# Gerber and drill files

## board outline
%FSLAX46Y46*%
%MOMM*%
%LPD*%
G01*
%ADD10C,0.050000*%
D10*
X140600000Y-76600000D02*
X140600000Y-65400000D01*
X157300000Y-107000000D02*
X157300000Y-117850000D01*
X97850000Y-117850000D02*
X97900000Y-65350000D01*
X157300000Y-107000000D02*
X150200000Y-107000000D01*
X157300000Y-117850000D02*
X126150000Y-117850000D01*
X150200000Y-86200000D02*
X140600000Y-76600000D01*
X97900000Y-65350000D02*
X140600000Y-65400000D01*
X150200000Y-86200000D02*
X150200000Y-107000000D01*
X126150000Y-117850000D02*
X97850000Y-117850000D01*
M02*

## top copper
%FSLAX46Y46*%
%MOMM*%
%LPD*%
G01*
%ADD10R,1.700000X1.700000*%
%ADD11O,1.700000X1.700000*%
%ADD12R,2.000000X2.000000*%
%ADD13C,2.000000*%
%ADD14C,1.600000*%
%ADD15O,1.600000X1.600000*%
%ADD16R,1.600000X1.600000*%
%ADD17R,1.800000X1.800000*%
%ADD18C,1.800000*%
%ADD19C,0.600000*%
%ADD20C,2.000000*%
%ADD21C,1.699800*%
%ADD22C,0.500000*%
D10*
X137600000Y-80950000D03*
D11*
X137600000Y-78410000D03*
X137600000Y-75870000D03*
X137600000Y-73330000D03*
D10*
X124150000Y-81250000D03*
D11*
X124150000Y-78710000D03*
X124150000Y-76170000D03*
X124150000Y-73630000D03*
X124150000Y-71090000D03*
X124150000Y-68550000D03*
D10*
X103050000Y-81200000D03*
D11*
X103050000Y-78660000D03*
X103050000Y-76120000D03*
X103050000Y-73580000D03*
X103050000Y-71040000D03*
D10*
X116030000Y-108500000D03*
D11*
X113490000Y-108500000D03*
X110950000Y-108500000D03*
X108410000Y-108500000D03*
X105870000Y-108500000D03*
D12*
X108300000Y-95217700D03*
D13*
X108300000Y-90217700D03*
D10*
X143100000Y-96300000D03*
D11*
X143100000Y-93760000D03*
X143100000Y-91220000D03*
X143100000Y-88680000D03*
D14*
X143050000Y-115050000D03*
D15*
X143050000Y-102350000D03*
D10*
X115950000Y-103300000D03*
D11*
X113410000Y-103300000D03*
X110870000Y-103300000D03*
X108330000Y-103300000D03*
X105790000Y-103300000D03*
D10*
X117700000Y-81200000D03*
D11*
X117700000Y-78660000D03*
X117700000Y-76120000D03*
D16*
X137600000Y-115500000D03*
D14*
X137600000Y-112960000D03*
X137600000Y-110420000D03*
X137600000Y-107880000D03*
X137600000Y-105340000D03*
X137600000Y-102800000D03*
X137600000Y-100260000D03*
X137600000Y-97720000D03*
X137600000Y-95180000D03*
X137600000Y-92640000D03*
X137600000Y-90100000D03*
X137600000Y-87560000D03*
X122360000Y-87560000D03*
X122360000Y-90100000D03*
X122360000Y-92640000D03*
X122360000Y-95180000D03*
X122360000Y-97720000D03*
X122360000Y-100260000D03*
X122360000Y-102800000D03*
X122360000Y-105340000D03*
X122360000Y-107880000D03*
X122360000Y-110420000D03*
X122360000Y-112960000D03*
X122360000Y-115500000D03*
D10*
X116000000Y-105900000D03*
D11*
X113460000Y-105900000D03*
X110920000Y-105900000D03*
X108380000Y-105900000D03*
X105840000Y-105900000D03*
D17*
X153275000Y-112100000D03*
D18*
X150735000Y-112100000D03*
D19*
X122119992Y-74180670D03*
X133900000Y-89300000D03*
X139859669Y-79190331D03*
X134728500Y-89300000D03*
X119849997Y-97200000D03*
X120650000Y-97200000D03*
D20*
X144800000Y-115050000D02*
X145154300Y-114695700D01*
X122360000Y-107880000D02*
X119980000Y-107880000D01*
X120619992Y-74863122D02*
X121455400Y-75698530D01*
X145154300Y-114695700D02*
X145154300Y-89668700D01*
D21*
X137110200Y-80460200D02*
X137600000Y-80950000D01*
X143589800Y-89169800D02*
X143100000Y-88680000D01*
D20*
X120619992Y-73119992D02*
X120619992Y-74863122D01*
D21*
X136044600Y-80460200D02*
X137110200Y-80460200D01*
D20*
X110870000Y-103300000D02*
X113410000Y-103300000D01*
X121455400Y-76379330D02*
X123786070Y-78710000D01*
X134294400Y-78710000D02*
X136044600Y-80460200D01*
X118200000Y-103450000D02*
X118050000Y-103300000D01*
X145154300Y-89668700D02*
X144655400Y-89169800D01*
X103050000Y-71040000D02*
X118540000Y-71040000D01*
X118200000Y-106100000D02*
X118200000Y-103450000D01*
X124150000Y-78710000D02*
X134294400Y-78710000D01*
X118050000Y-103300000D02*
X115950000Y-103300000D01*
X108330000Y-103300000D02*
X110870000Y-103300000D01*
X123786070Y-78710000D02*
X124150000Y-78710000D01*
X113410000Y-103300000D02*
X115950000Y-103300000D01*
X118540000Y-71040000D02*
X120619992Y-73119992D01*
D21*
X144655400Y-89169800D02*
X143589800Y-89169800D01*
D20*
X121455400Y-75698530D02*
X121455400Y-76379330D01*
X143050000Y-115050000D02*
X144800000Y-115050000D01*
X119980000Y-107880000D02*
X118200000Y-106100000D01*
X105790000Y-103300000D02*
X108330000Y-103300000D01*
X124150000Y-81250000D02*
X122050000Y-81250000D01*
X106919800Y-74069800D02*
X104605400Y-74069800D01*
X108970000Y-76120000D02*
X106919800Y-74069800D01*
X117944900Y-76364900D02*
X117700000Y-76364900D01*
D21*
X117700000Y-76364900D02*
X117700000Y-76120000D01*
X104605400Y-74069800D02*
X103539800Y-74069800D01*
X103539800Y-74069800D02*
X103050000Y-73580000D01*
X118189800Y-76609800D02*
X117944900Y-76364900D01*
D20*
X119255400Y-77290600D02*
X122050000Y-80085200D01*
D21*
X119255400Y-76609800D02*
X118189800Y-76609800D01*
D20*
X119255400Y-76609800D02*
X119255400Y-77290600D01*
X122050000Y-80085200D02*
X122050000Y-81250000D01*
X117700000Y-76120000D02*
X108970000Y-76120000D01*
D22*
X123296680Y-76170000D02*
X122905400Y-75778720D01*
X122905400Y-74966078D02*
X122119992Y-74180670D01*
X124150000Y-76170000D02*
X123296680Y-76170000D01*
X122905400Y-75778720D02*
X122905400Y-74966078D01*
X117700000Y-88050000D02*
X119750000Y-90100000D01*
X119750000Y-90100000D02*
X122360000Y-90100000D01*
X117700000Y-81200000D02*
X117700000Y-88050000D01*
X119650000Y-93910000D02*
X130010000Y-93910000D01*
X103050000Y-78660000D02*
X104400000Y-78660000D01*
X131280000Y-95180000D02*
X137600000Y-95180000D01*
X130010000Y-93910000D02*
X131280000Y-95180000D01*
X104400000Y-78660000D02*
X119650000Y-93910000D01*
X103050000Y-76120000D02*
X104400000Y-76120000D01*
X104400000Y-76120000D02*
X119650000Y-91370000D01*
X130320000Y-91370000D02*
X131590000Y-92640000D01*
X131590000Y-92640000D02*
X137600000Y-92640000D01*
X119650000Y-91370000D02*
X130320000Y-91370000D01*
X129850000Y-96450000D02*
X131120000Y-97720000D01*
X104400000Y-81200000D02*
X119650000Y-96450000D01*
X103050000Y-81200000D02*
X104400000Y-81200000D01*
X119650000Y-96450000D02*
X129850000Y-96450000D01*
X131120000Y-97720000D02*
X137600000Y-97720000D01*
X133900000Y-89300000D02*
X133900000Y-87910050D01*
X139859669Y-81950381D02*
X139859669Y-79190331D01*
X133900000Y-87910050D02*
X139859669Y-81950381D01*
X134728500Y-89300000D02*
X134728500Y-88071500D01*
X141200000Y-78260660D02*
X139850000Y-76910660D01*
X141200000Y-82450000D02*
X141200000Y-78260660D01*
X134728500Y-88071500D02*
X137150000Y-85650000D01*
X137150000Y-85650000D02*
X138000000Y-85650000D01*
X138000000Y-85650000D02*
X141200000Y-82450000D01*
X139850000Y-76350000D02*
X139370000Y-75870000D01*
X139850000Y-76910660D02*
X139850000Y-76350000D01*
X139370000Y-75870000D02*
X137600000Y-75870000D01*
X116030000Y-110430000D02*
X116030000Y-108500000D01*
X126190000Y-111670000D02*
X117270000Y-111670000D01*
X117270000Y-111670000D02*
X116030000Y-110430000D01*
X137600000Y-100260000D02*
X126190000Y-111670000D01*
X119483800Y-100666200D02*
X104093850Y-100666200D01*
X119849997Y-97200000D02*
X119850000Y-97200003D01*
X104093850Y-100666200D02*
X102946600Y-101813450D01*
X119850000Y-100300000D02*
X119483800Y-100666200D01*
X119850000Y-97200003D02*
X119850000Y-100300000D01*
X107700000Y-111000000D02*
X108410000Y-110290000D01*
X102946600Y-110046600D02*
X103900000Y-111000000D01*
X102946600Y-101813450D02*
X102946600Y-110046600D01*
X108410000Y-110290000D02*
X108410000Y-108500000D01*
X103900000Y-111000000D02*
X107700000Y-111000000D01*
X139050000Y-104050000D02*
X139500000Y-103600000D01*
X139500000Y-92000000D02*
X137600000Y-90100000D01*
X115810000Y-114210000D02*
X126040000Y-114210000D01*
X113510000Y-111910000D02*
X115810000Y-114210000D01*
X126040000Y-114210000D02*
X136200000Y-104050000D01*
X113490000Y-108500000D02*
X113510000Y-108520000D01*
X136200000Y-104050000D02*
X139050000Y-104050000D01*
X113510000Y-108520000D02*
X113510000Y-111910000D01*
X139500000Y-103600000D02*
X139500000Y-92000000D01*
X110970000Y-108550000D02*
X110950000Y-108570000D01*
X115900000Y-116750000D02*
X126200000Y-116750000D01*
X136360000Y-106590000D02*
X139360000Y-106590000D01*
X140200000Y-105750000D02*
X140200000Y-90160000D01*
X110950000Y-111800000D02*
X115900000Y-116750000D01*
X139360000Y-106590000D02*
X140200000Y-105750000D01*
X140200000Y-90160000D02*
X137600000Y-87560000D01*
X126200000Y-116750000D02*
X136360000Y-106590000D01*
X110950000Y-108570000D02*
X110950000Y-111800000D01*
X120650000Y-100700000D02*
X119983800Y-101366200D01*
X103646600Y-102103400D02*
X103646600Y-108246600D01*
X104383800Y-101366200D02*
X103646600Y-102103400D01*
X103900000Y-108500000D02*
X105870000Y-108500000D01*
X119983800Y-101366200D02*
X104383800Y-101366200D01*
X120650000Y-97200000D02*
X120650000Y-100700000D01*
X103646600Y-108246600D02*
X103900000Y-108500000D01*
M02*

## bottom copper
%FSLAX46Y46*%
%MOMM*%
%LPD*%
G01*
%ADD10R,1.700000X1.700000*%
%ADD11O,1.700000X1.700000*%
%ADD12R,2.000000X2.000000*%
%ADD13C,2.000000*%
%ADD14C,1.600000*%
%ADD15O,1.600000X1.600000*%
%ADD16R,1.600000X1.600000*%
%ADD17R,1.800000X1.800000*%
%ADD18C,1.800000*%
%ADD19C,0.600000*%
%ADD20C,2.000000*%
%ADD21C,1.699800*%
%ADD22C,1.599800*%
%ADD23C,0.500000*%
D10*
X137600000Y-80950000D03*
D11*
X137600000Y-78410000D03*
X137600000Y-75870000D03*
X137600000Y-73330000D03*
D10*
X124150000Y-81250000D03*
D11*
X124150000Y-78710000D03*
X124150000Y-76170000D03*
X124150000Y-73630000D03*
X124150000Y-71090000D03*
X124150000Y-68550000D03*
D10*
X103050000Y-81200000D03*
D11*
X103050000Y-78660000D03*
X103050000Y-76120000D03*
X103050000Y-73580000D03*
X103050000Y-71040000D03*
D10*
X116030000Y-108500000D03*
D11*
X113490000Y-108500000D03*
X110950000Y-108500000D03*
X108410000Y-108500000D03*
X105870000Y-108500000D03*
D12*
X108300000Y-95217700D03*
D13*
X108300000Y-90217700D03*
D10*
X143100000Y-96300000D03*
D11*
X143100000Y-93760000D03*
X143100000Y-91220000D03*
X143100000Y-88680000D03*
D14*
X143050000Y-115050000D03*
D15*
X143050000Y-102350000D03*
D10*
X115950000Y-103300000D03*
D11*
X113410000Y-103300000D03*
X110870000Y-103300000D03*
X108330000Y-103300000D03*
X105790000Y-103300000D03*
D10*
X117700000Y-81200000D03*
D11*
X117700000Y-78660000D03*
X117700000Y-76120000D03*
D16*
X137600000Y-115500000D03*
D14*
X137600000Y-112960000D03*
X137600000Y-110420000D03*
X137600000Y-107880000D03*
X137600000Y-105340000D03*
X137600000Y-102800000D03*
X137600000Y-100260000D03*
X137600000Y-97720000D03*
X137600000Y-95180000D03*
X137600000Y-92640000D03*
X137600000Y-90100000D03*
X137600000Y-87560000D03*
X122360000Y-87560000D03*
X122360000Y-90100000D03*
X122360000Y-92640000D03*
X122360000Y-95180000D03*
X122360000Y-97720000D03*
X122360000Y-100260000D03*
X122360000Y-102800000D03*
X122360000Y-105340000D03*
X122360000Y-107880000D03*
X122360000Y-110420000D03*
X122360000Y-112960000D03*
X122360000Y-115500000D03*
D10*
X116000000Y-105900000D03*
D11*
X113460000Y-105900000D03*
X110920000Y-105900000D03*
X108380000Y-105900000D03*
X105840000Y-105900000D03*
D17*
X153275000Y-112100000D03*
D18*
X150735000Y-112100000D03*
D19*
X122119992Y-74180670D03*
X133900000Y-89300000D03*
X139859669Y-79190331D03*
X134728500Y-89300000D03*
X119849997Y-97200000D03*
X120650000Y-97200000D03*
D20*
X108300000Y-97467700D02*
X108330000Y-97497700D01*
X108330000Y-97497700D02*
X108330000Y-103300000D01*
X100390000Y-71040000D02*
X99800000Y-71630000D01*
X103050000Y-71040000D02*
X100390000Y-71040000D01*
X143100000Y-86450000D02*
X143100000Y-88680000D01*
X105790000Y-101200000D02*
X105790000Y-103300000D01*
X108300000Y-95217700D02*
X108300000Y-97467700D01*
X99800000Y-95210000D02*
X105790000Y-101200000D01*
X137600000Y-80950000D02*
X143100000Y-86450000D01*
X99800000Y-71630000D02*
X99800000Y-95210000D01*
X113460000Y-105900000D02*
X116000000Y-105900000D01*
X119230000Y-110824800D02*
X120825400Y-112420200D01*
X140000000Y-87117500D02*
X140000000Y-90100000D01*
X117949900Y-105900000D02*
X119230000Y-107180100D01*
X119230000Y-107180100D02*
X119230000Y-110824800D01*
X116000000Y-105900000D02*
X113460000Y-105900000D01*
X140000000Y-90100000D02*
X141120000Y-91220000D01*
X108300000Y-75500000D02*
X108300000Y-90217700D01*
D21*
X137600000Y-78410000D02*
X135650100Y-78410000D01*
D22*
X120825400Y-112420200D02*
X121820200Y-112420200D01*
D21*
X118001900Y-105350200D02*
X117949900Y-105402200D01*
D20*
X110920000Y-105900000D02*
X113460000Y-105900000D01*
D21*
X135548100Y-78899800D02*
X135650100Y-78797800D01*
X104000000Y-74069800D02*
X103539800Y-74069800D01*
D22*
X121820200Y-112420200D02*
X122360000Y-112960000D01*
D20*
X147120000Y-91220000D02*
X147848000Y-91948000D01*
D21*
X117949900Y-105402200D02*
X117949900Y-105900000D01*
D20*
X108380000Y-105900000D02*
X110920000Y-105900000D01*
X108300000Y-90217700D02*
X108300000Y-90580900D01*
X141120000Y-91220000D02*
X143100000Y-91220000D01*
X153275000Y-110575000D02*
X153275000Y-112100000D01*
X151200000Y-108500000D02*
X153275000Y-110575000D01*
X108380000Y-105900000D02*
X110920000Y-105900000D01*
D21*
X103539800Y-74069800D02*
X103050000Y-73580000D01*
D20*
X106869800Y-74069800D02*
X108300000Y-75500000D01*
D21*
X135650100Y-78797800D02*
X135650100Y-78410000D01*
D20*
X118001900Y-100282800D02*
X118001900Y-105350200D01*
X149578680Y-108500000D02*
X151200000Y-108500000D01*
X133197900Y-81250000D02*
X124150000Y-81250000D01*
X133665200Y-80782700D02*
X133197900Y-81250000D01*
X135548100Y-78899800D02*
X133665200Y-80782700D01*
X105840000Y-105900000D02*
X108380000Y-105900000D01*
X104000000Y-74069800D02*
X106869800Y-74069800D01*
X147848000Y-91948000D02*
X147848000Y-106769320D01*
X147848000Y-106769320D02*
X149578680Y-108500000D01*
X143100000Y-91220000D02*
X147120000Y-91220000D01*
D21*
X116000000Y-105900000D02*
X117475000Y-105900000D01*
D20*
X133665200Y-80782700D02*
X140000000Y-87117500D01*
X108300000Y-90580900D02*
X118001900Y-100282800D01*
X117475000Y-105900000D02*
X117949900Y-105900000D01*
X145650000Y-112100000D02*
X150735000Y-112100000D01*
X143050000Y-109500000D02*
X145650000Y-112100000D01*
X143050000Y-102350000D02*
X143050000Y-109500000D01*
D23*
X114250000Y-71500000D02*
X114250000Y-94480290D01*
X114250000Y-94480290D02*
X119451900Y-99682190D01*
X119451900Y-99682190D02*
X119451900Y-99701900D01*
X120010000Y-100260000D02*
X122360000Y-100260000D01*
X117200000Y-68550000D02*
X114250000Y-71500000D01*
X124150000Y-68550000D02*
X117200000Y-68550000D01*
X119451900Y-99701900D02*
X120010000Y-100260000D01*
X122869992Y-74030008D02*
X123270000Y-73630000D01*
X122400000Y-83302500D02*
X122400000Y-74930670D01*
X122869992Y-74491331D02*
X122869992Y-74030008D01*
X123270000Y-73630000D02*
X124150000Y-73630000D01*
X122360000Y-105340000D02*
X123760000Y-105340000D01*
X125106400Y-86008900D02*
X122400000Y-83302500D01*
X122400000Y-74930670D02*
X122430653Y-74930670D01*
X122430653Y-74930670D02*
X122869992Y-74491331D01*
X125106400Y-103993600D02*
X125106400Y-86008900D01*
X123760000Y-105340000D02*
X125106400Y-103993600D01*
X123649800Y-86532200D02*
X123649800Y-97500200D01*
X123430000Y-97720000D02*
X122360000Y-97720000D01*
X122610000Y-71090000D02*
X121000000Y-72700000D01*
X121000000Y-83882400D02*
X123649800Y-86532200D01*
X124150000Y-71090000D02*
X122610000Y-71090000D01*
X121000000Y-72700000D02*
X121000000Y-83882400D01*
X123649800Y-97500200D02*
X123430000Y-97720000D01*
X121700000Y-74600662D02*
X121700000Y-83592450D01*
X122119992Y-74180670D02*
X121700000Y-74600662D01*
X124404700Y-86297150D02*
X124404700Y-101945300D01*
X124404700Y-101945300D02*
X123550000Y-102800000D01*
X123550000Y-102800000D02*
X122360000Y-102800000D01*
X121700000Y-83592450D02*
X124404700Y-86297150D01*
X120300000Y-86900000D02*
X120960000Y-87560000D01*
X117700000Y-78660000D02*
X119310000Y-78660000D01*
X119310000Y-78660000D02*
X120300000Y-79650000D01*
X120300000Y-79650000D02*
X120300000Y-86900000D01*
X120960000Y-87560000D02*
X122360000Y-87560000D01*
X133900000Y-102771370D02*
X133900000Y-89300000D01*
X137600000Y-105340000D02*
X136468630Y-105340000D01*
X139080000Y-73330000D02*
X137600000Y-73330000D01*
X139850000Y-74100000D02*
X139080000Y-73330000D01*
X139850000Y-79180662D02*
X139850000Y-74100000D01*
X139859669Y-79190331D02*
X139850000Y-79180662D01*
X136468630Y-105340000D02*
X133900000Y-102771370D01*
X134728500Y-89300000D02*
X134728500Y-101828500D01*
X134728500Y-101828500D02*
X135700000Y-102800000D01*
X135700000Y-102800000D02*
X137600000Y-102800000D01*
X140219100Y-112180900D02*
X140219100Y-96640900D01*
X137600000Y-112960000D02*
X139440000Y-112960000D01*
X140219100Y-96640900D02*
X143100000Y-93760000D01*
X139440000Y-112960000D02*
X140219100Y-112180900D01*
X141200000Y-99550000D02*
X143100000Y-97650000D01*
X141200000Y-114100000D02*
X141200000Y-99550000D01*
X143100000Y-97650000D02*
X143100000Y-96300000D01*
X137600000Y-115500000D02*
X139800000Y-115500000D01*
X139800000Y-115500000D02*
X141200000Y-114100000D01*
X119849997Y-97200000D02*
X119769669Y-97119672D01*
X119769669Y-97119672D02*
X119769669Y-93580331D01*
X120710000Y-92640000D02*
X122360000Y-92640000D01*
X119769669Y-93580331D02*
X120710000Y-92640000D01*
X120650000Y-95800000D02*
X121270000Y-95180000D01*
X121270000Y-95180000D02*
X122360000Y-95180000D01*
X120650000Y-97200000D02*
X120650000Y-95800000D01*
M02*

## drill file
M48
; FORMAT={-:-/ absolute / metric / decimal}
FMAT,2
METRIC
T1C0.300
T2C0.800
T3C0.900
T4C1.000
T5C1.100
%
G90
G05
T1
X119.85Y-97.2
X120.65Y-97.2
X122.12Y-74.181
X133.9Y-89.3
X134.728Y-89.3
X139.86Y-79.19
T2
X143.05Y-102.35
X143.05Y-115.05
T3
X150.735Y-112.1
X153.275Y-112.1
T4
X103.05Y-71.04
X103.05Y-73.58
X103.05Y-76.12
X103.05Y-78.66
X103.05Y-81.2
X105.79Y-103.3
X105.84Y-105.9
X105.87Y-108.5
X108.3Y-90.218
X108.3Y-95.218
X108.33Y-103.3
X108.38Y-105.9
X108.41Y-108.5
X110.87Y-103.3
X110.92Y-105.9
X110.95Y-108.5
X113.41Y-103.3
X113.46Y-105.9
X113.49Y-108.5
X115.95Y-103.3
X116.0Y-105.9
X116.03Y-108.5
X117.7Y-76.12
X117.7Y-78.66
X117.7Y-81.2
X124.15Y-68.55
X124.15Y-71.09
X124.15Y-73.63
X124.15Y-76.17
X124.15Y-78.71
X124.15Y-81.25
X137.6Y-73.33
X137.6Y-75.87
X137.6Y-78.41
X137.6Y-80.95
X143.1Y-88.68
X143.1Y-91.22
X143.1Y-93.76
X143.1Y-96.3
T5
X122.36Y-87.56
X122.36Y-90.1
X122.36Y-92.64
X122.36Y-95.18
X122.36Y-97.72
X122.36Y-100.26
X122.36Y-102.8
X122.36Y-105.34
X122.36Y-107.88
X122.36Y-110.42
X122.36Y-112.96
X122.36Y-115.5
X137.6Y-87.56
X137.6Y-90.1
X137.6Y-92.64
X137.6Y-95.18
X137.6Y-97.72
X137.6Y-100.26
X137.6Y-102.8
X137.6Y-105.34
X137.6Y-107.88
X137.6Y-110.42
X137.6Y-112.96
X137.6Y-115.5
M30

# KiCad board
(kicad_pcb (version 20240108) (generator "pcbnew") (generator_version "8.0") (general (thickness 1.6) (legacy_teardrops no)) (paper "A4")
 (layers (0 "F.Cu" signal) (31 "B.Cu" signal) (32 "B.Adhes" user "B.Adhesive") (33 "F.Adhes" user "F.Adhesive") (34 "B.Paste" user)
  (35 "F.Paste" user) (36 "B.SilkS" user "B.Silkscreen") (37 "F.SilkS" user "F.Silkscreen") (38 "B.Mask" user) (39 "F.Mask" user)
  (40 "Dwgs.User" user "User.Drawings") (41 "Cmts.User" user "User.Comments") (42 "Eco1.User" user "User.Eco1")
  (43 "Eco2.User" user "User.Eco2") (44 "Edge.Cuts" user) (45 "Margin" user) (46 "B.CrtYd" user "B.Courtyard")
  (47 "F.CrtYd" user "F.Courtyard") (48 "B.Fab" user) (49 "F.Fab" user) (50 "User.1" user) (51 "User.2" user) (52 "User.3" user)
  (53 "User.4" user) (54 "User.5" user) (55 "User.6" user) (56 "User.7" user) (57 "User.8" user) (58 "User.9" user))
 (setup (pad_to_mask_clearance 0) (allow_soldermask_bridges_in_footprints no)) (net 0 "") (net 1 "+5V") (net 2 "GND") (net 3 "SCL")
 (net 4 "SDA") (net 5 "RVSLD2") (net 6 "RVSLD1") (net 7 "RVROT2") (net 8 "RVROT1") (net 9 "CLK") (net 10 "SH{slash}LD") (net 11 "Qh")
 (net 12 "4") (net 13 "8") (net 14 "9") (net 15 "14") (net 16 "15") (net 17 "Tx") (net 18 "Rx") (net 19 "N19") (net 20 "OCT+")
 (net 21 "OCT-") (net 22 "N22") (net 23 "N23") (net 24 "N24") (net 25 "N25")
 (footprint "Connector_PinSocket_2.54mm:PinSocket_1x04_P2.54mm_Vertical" (layer "F.Cu") (at 137.6 80.95 180)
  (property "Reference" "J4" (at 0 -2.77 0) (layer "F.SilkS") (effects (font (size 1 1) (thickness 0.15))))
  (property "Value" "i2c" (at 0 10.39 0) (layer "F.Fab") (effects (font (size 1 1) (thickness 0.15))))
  (pad "1" thru_hole rect (at 0 0 180) (size 1.7 1.7) (drill 1) (layers "*.Cu" "*.Mask") (remove_unused_layers no) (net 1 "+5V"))
  (pad "2" thru_hole oval (at 0 2.54 180) (size 1.7 1.7) (drill 1) (layers "*.Cu" "*.Mask") (remove_unused_layers no) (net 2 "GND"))
  (pad "3" thru_hole oval (at 0 5.08 180) (size 1.7 1.7) (drill 1) (layers "*.Cu" "*.Mask") (remove_unused_layers no) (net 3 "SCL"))
  (pad "4" thru_hole oval (at 0 7.62 180) (size 1.7 1.7) (drill 1) (layers "*.Cu" "*.Mask") (remove_unused_layers no) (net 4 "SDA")))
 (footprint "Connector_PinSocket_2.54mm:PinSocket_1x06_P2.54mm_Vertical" (layer "F.Cu") (at 124.15 81.25 180)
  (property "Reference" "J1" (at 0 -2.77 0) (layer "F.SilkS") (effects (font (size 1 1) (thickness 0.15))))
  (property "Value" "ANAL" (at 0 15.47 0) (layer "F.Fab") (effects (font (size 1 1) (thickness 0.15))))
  (pad "1" thru_hole rect (at 0 0 180) (size 1.7 1.7) (drill 1) (layers "*.Cu" "*.Mask") (remove_unused_layers no) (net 2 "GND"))
  (pad "2" thru_hole oval (at 0 2.54 180) (size 1.7 1.7) (drill 1) (layers "*.Cu" "*.Mask") (remove_unused_layers no) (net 1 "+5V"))
  (pad "3" thru_hole oval (at 0 5.08 180) (size 1.7 1.7) (drill 1) (layers "*.Cu" "*.Mask") (remove_unused_layers no) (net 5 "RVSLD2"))
  (pad "4" thru_hole oval (at 0 7.62 180) (size 1.7 1.7) (drill 1) (layers "*.Cu" "*.Mask") (remove_unused_layers no) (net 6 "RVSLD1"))
  (pad "5" thru_hole oval (at 0 10.16 180) (size 1.7 1.7) (drill 1) (layers "*.Cu" "*.Mask") (remove_unused_layers no) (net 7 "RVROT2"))
  (pad "6" thru_hole oval (at 0 12.7 180) (size 1.7 1.7) (drill 1) (layers "*.Cu" "*.Mask") (remove_unused_layers no) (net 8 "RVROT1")))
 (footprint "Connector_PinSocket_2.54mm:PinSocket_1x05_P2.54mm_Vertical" (layer "F.Cu") (at 103.05 81.2 180)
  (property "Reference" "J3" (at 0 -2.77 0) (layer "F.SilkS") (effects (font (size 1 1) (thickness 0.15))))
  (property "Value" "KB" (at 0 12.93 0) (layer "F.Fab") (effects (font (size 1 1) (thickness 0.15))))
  (pad "1" thru_hole rect (at 0 0 180) (size 1.7 1.7) (drill 1) (layers "*.Cu" "*.Mask") (remove_unused_layers no) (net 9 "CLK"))
  (pad "2" thru_hole oval (at 0 2.54 180) (size 1.7 1.7) (drill 1) (layers "*.Cu" "*.Mask") (remove_unused_layers no) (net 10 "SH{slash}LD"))
  (pad "3" thru_hole oval (at 0 5.08 180) (size 1.7 1.7) (drill 1) (layers "*.Cu" "*.Mask") (remove_unused_layers no) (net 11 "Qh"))
  (pad "4" thru_hole oval (at 0 7.62 180) (size 1.7 1.7) (drill 1) (layers "*.Cu" "*.Mask") (remove_unused_layers no) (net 2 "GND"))
  (pad "5" thru_hole oval (at 0 10.16 180) (size 1.7 1.7) (drill 1) (layers "*.Cu" "*.Mask") (remove_unused_layers no) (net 1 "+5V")))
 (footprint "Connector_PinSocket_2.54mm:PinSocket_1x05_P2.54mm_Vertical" (layer "F.Cu") (at 116.03 108.5 -90)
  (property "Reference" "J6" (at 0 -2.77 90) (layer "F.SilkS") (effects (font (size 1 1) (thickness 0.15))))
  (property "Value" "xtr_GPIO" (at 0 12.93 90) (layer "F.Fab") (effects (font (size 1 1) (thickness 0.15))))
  (pad "1" thru_hole rect (at 0 0 270) (size 1.7 1.7) (drill 1) (layers "*.Cu" "*.Mask") (remove_unused_layers no) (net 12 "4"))
  (pad "2" thru_hole oval (at 0 2.54 270) (size 1.7 1.7) (drill 1) (layers "*.Cu" "*.Mask") (remove_unused_layers no) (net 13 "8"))
  (pad "3" thru_hole oval (at 0 5.08 270) (size 1.7 1.7) (drill 1) (layers "*.Cu" "*.Mask") (remove_unused_layers no) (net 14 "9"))
  (pad "4" thru_hole oval (at 0 7.62 270) (size 1.7 1.7) (drill 1) (layers "*.Cu" "*.Mask") (remove_unused_layers no) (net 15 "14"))
  (pad "5" thru_hole oval (at 0 10.16 270) (size 1.7 1.7) (drill 1) (layers "*.Cu" "*.Mask") (remove_unused_layers no) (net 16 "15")))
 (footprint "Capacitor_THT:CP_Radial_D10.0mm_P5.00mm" (layer "F.Cu") (at 108.3 95.2177 90)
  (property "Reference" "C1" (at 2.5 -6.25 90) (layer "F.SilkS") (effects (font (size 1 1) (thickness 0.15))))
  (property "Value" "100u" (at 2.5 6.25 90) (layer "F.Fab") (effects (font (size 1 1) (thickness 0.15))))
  (pad "1" thru_hole rect (at 0 0 90) (size 2 2) (drill 1) (layers "*.Cu" "*.Mask") (remove_unused_layers no) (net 1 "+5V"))
  (pad "2" thru_hole circle (at 5 0 90) (size 2 2) (drill 1) (layers "*.Cu" "*.Mask") (remove_unused_layers no) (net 2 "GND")))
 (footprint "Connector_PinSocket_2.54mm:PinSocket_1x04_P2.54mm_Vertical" (layer "F.Cu") (at 143.1 96.3 180)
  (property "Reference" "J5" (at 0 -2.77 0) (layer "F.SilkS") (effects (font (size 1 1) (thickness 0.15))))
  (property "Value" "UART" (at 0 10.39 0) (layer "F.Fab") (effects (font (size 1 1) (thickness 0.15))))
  (pad "1" thru_hole rect (at 0 0 180) (size 1.7 1.7) (drill 1) (layers "*.Cu" "*.Mask") (remove_unused_layers no) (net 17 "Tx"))
  (pad "2" thru_hole oval (at 0 2.54 180) (size 1.7 1.7) (drill 1) (layers "*.Cu" "*.Mask") (remove_unused_layers no) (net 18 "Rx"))
  (pad "3" thru_hole oval (at 0 5.08 180) (size 1.7 1.7) (drill 1) (layers "*.Cu" "*.Mask") (remove_unused_layers no) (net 2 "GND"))
  (pad "4" thru_hole oval (at 0 7.62 180) (size 1.7 1.7) (drill 1) (layers "*.Cu" "*.Mask") (remove_unused_layers no) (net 1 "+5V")))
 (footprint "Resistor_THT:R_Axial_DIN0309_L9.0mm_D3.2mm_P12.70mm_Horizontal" (layer "F.Cu") (at 143.05 115.05 90)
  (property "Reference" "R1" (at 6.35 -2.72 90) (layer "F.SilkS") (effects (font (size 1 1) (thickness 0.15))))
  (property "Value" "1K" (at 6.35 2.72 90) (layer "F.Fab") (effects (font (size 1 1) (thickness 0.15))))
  (pad "1" thru_hole circle (at 0 0 90) (size 1.6 1.6) (drill 0.8) (layers "*.Cu" "*.Mask") (remove_unused_layers no) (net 1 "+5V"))
  (pad "2" thru_hole oval (at 12.7 0 90) (size 1.6 1.6) (drill 0.8) (layers "*.Cu" "*.Mask") (remove_unused_layers no) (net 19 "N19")))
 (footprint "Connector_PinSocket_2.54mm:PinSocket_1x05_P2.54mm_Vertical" (layer "F.Cu") (at 115.95 103.3 -90)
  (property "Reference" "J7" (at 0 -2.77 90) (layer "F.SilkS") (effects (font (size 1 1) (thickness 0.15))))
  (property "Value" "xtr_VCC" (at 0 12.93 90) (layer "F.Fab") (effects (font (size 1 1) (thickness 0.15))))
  (pad "1" thru_hole rect (at 0 0 270) (size 1.7 1.7) (drill 1) (layers "*.Cu" "*.Mask") (remove_unused_layers no) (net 1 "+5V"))
  (pad "2" thru_hole oval (at 0 2.54 270) (size 1.7 1.7) (drill 1) (layers "*.Cu" "*.Mask") (remove_unused_layers no) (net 1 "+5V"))
  (pad "3" thru_hole oval (at 0 5.08 270) (size 1.7 1.7) (drill 1) (layers "*.Cu" "*.Mask") (remove_unused_layers no) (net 1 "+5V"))
  (pad "4" thru_hole oval (at 0 7.62 270) (size 1.7 1.7) (drill 1) (layers "*.Cu" "*.Mask") (remove_unused_layers no) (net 1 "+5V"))
  (pad "5" thru_hole oval (at 0 10.16 270) (size 1.7 1.7) (drill 1) (layers "*.Cu" "*.Mask") (remove_unused_layers no) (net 1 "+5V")))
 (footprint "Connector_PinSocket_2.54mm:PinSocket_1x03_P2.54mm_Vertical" (layer "F.Cu") (at 117.7 81.2 180)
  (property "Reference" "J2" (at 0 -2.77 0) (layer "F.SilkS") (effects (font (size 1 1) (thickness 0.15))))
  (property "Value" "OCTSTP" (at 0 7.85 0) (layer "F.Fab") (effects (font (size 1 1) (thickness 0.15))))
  (pad "1" thru_hole rect (at 0 0 180) (size 1.7 1.7) (drill 1) (layers "*.Cu" "*.Mask") (remove_unused_layers no) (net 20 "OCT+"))
  (pad "2" thru_hole oval (at 0 2.54 180) (size 1.7 1.7) (drill 1) (layers "*.Cu" "*.Mask") (remove_unused_layers no) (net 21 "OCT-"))
  (pad "3" thru_hole oval (at 0 5.08 180) (size 1.7 1.7) (drill 1) (layers "*.Cu" "*.Mask") (remove_unused_layers no) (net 2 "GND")))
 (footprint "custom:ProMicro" (layer "F.Cu") (at 129.98 101.53 90)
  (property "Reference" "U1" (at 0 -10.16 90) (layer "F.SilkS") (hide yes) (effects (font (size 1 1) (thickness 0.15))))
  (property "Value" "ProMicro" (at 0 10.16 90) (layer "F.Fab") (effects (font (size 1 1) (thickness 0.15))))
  (pad "1" thru_hole rect (at -13.97 7.62 90) (size 1.6 1.6) (drill 1.1) (layers "*.Cu" "*.Mask" "F.SilkS") (remove_unused_layers no)
   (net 17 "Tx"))
  (pad "2" thru_hole circle (at -11.43 7.62 90) (size 1.6 1.6) (drill 1.1) (layers "*.Cu" "*.Mask" "F.SilkS") (remove_unused_layers no)
   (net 18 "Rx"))
  (pad "3" thru_hole circle (at -8.89 7.62 90) (size 1.6 1.6) (drill 1.1) (layers "*.Cu" "*.Mask" "F.SilkS") (remove_unused_layers no)
   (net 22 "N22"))
  (pad "4" thru_hole circle (at -6.35 7.62 90) (size 1.6 1.6) (drill 1.1) (layers "*.Cu" "*.Mask" "F.SilkS") (remove_unused_layers no)
   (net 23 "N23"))
  (pad "5" thru_hole circle (at -3.81 7.62 90) (size 1.6 1.6) (drill 1.1) (layers "*.Cu" "*.Mask" "F.SilkS") (remove_unused_layers no)
   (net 4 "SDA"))
  (pad "6" thru_hole circle (at -1.27 7.62 90) (size 1.6 1.6) (drill 1.1) (layers "*.Cu" "*.Mask" "F.SilkS") (remove_unused_layers no)
   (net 3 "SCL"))
  (pad "7" thru_hole circle (at 1.27 7.62 90) (size 1.6 1.6) (drill 1.1) (layers "*.Cu" "*.Mask" "F.SilkS") (remove_unused_layers no)
   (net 12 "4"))
  (pad "8" thru_hole circle (at 3.81 7.62 90) (size 1.6 1.6) (drill 1.1) (layers "*.Cu" "*.Mask" "F.SilkS") (remove_unused_layers no)
   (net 9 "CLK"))
  (pad "9" thru_hole circle (at 6.35 7.62 90) (size 1.6 1.6) (drill 1.1) (layers "*.Cu" "*.Mask" "F.SilkS") (remove_unused_layers no)
   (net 10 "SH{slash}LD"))
  (pad "10" thru_hole circle (at 8.89 7.62 90) (size 1.6 1.6) (drill 1.1) (layers "*.Cu" "*.Mask" "F.SilkS") (remove_unused_layers no)
   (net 11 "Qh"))
  (pad "11" thru_hole circle (at 11.43 7.62 90) (size 1.6 1.6) (drill 1.1) (layers "*.Cu" "*.Mask" "F.SilkS") (remove_unused_layers no)
   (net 13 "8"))
  (pad "12" thru_hole circle (at 13.97 7.62 90) (size 1.6 1.6) (drill 1.1) (layers "*.Cu" "*.Mask" "F.SilkS") (remove_unused_layers no)
   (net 14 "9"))
  (pad "13" thru_hole circle (at 13.97 -7.62 90) (size 1.6 1.6) (drill 1.1) (layers "*.Cu" "*.Mask" "F.SilkS") (remove_unused_layers no)
   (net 21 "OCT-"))
  (pad "14" thru_hole circle (at 11.43 -7.62 90) (size 1.6 1.6) (drill 1.1) (layers "*.Cu" "*.Mask" "F.SilkS") (remove_unused_layers no)
   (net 20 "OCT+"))
  (pad "15" thru_hole circle (at 8.89 -7.62 90) (size 1.6 1.6) (drill 1.1) (layers "*.Cu" "*.Mask" "F.SilkS") (remove_unused_layers no)
   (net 15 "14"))
  (pad "16" thru_hole circle (at 6.35 -7.62 90) (size 1.6 1.6) (drill 1.1) (layers "*.Cu" "*.Mask" "F.SilkS") (remove_unused_layers no)
   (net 16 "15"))
  (pad "17" thru_hole circle (at 3.81 -7.62 90) (size 1.6 1.6) (drill 1.1) (layers "*.Cu" "*.Mask" "F.SilkS") (remove_unused_layers no)
   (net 7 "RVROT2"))
  (pad "18" thru_hole circle (at 1.27 -7.62 90) (size 1.6 1.6) (drill 1.1) (layers "*.Cu" "*.Mask" "F.SilkS") (remove_unused_layers no)
   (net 8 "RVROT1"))
  (pad "19" thru_hole circle (at -1.27 -7.62 90) (size 1.6 1.6) (drill 1.1) (layers "*.Cu" "*.Mask" "F.SilkS") (remove_unused_layers no)
   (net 5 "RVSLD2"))
  (pad "20" thru_hole circle (at -3.81 -7.62 90) (size 1.6 1.6) (drill 1.1) (layers "*.Cu" "*.Mask" "F.SilkS") (remove_unused_layers no)
   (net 6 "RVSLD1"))
  (pad "21" thru_hole circle (at -6.35 -7.62 90) (size 1.6 1.6) (drill 1.1) (layers "*.Cu" "*.Mask" "F.SilkS") (remove_unused_layers no)
   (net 1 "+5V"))
  (pad "22" thru_hole circle (at -8.89 -7.62 90) (size 1.6 1.6) (drill 1.1) (layers "*.Cu" "*.Mask" "F.SilkS") (remove_unused_layers no)
   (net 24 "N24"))
  (pad "23" thru_hole circle (at -11.43 -7.62 90) (size 1.6 1.6) (drill 1.1) (layers "*.Cu" "*.Mask" "F.SilkS") (remove_unused_layers no)
   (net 2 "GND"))
  (pad "24" thru_hole circle (at -13.97 -7.62 90) (size 1.6 1.6) (drill 1.1) (layers "*.Cu" "*.Mask" "F.SilkS") (remove_unused_layers no)
   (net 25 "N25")))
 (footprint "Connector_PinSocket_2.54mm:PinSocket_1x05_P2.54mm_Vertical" (layer "F.Cu") (at 116 105.9 -90)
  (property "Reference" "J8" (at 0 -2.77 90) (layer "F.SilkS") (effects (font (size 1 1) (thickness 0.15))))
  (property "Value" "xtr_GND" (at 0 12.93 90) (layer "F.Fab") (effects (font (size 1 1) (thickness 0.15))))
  (pad "1" thru_hole rect (at 0 0 270) (size 1.7 1.7) (drill 1) (layers "*.Cu" "*.Mask") (remove_unused_layers no) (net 2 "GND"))
  (pad "2" thru_hole oval (at 0 2.54 270) (size 1.7 1.7) (drill 1) (layers "*.Cu" "*.Mask") (remove_unused_layers no) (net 2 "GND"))
  (pad "3" thru_hole oval (at 0 5.08 270) (size 1.7 1.7) (drill 1) (layers "*.Cu" "*.Mask") (remove_unused_layers no) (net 2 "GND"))
  (pad "4" thru_hole oval (at 0 7.62 270) (size 1.7 1.7) (drill 1) (layers "*.Cu" "*.Mask") (remove_unused_layers no) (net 2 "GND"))
  (pad "5" thru_hole oval (at 0 10.16 270) (size 1.7 1.7) (drill 1) (layers "*.Cu" "*.Mask") (remove_unused_layers no) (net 2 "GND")))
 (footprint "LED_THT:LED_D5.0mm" (layer "F.Cu") (at 153.275 112.1 180)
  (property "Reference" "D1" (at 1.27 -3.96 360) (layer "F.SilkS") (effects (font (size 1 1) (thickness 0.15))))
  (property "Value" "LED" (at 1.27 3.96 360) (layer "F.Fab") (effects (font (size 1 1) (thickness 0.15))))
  (pad "1" thru_hole rect (at 0 0 180) (size 1.8 1.8) (drill 0.9) (layers "*.Cu" "*.Mask") (remove_unused_layers no) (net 2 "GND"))
  (pad "2" thru_hole circle (at 2.54 0 180) (size 1.8 1.8) (drill 0.9) (layers "*.Cu" "*.Mask") (remove_unused_layers no) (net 19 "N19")))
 (gr_line (start 140.6 76.6) (end 140.6 65.4) (stroke (width 0.05) (type default)) (layer "Edge.Cuts"))
 (gr_line (start 157.3 107) (end 157.3 117.85) (stroke (width 0.05) (type default)) (layer "Edge.Cuts"))
 (gr_line (start 97.85 117.85) (end 97.9 65.35) (stroke (width 0.05) (type default)) (layer "Edge.Cuts"))
 (gr_line (start 157.3 107) (end 150.2 107) (stroke (width 0.05) (type default)) (layer "Edge.Cuts"))
 (gr_line (start 157.3 117.85) (end 126.15 117.85) (stroke (width 0.05) (type default)) (layer "Edge.Cuts"))
 (gr_line (start 150.2 86.2) (end 140.6 76.6) (stroke (width 0.05) (type default)) (layer "Edge.Cuts"))
 (gr_line (start 97.9 65.35) (end 140.6 65.4) (stroke (width 0.05) (type default)) (layer "Edge.Cuts"))
 (gr_line (start 150.2 86.2) (end 150.2 107) (stroke (width 0.05) (type default)) (layer "Edge.Cuts"))
 (gr_line (start 126.15 117.85) (end 97.85 117.85) (stroke (width 0.05) (type default)) (layer "Edge.Cuts"))
 (segment (start 144.8 115.05) (end 145.1543 114.6957) (width 2) (layer "F.Cu") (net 1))
 (segment (start 122.36 107.88) (end 119.98 107.88) (width 2) (layer "F.Cu") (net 1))
 (segment (start 120.619992 74.863122) (end 121.4554 75.69853) (width 2) (layer "F.Cu") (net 1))
 (segment (start 145.1543 114.6957) (end 145.1543 89.6687) (width 2) (layer "F.Cu") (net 1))
 (segment (start 137.1102 80.4602) (end 137.6 80.95) (width 1.6998) (layer "F.Cu") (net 1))
 (segment (start 143.5898 89.1698) (end 143.1 88.68) (width 1.6998) (layer "F.Cu") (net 1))
 (segment (start 120.619992 73.119992) (end 120.619992 74.863122) (width 2) (layer "F.Cu") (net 1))
 (segment (start 136.0446 80.4602) (end 137.1102 80.4602) (width 1.6998) (layer "F.Cu") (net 1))
 (segment (start 110.87 103.3) (end 113.41 103.3) (width 2) (layer "F.Cu") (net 1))
 (segment (start 121.4554 76.37933) (end 123.78607 78.71) (width 2) (layer "F.Cu") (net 1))
 (segment (start 134.2944 78.71) (end 136.0446 80.4602) (width 2) (layer "F.Cu") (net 1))
 (segment (start 118.2 103.45) (end 118.05 103.3) (width 2) (layer "F.Cu") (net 1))
 (segment (start 145.1543 89.6687) (end 144.6554 89.1698) (width 2) (layer "F.Cu") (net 1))
 (segment (start 103.05 71.04) (end 118.54 71.04) (width 2) (layer "F.Cu") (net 1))
 (segment (start 118.2 106.1) (end 118.2 103.45) (width 2) (layer "F.Cu") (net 1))
 (segment (start 124.15 78.71) (end 134.2944 78.71) (width 2) (layer "F.Cu") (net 1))
 (segment (start 118.05 103.3) (end 115.95 103.3) (width 2) (layer "F.Cu") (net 1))
 (segment (start 108.33 103.3) (end 110.87 103.3) (width 2) (layer "F.Cu") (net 1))
 (segment (start 123.78607 78.71) (end 124.15 78.71) (width 2) (layer "F.Cu") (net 1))
 (segment (start 113.41 103.3) (end 115.95 103.3) (width 2) (layer "F.Cu") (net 1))
 (segment (start 118.54 71.04) (end 120.619992 73.119992) (width 2) (layer "F.Cu") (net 1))
 (segment (start 144.6554 89.1698) (end 143.5898 89.1698) (width 1.6998) (layer "F.Cu") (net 1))
 (segment (start 121.4554 75.69853) (end 121.4554 76.37933) (width 2) (layer "F.Cu") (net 1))
 (segment (start 143.05 115.05) (end 144.8 115.05) (width 2) (layer "F.Cu") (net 1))
 (segment (start 119.98 107.88) (end 118.2 106.1) (width 2) (layer "F.Cu") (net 1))
 (segment (start 105.79 103.3) (end 108.33 103.3) (width 2) (layer "F.Cu") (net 1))
 (segment (start 108.3 97.4677) (end 108.33 97.4977) (width 2) (layer "B.Cu") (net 1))
 (segment (start 108.33 97.4977) (end 108.33 103.3) (width 2) (layer "B.Cu") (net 1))
 (segment (start 100.39 71.04) (end 99.8 71.63) (width 2) (layer "B.Cu") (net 1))
 (segment (start 103.05 71.04) (end 100.39 71.04) (width 2) (layer "B.Cu") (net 1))
 (segment (start 143.1 86.45) (end 143.1 88.68) (width 2) (layer "B.Cu") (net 1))
 (segment (start 105.79 101.2) (end 105.79 103.3) (width 2) (layer "B.Cu") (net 1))
 (segment (start 108.3 95.2177) (end 108.3 97.4677) (width 2) (layer "B.Cu") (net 1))
 (segment (start 99.8 95.21) (end 105.79 101.2) (width 2) (layer "B.Cu") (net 1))
 (segment (start 137.6 80.95) (end 143.1 86.45) (width 2) (layer "B.Cu") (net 1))
 (segment (start 99.8 71.63) (end 99.8 95.21) (width 2) (layer "B.Cu") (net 1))
 (segment (start 124.15 81.25) (end 122.05 81.25) (width 2) (layer "F.Cu") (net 2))
 (segment (start 106.9198 74.0698) (end 104.6054 74.0698) (width 2) (layer "F.Cu") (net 2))
 (segment (start 108.97 76.12) (end 106.9198 74.0698) (width 2) (layer "F.Cu") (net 2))
 (segment (start 117.9449 76.3649) (end 117.7 76.3649) (width 2) (layer "F.Cu") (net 2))
 (segment (start 117.7 76.3649) (end 117.7 76.12) (width 1.6998) (layer "F.Cu") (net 2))
 (segment (start 104.6054 74.0698) (end 103.5398 74.0698) (width 1.6998) (layer "F.Cu") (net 2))
 (segment (start 103.5398 74.0698) (end 103.05 73.58) (width 1.6998) (layer "F.Cu") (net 2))
 (segment (start 118.1898 76.6098) (end 117.9449 76.3649) (width 1.6998) (layer "F.Cu") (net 2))
 (segment (start 119.2554 77.2906) (end 122.05 80.0852) (width 2) (layer "F.Cu") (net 2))
 (segment (start 119.2554 76.6098) (end 118.1898 76.6098) (width 1.6998) (layer "F.Cu") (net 2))
 (segment (start 119.2554 76.6098) (end 119.2554 77.2906) (width 2) (layer "F.Cu") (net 2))
 (segment (start 122.05 80.0852) (end 122.05 81.25) (width 2) (layer "F.Cu") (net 2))
 (segment (start 117.7 76.12) (end 108.97 76.12) (width 2) (layer "F.Cu") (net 2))
 (segment (start 113.46 105.9) (end 116 105.9) (width 2) (layer "B.Cu") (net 2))
 (segment (start 119.23 110.8248) (end 120.8254 112.4202) (width 2) (layer "B.Cu") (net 2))
 (segment (start 140 87.1175) (end 140 90.1) (width 2) (layer "B.Cu") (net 2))
 (segment (start 117.9499 105.9) (end 119.23 107.1801) (width 2) (layer "B.Cu") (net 2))
 (segment (start 119.23 107.1801) (end 119.23 110.8248) (width 2) (layer "B.Cu") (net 2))
 (segment (start 116 105.9) (end 113.46 105.9) (width 2) (layer "B.Cu") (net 2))
 (segment (start 140 90.1) (end 141.12 91.22) (width 2) (layer "B.Cu") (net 2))
 (segment (start 108.3 75.5) (end 108.3 90.2177) (width 2) (layer "B.Cu") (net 2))
 (segment (start 137.6 78.41) (end 135.6501 78.41) (width 1.6998) (layer "B.Cu") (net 2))
 (segment (start 120.8254 112.4202) (end 121.8202 112.4202) (width 1.5998) (layer "B.Cu") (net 2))
 (segment (start 118.0019 105.3502) (end 117.9499 105.4022) (width 1.6998) (layer "B.Cu") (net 2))
 (segment (start 110.92 105.9) (end 113.46 105.9) (width 2) (layer "B.Cu") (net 2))
 (segment (start 135.5481 78.8998) (end 135.6501 78.7978) (width 1.6998) (layer "B.Cu") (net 2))
 (segment (start 104 74.0698) (end 103.5398 74.0698) (width 1.6998) (layer "B.Cu") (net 2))
 (segment (start 121.8202 112.4202) (end 122.36 112.96) (width 1.5998) (layer "B.Cu") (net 2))
 (segment (start 147.12 91.22) (end 147.848 91.948) (width 2) (layer "B.Cu") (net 2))
 (segment (start 117.9499 105.4022) (end 117.9499 105.9) (width 1.6998) (layer "B.Cu") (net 2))
 (segment (start 108.38 105.9) (end 110.92 105.9) (width 2) (layer "B.Cu") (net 2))
 (segment (start 108.3 90.2177) (end 108.3 90.5809) (width 2) (layer "B.Cu") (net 2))
 (segment (start 141.12 91.22) (end 143.1 91.22) (width 2) (layer "B.Cu") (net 2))
 (segment (start 153.275 110.575) (end 153.275 112.1) (width 2) (layer "B.Cu") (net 2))
 (segment (start 151.2 108.5) (end 153.275 110.575) (width 2) (layer "B.Cu") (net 2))
 (segment (start 108.38 105.9) (end 110.92 105.9) (width 2) (layer "B.Cu") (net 2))
 (segment (start 103.5398 74.0698) (end 103.05 73.58) (width 1.6998) (layer "B.Cu") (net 2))
 (segment (start 106.8698 74.0698) (end 108.3 75.5) (width 2) (layer "B.Cu") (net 2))
 (segment (start 135.6501 78.7978) (end 135.6501 78.41) (width 1.6998) (layer "B.Cu") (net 2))
 (segment (start 118.0019 100.2828) (end 118.0019 105.3502) (width 2) (layer "B.Cu") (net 2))
 (segment (start 149.57868 108.5) (end 151.2 108.5) (width 2) (layer "B.Cu") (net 2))
 (segment (start 133.1979 81.25) (end 124.15 81.25) (width 2) (layer "B.Cu") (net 2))
 (segment (start 133.6652 80.7827) (end 133.1979 81.25) (width 2) (layer "B.Cu") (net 2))
 (segment (start 135.5481 78.8998) (end 133.6652 80.7827) (width 2) (layer "B.Cu") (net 2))
 (segment (start 105.84 105.9) (end 108.38 105.9) (width 2) (layer "B.Cu") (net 2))
 (segment (start 104 74.0698) (end 106.8698 74.0698) (width 2) (layer "B.Cu") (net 2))
 (segment (start 147.848 91.948) (end 147.848 106.76932) (width 2) (layer "B.Cu") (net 2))
 (segment (start 147.848 106.76932) (end 149.57868 108.5) (width 2) (layer "B.Cu") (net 2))
 (segment (start 143.1 91.22) (end 147.12 91.22) (width 2) (layer "B.Cu") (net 2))
 (segment (start 116 105.9) (end 117.475 105.9) (width 1.6998) (layer "B.Cu") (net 2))
 (segment (start 133.6652 80.7827) (end 140 87.1175) (width 2) (layer "B.Cu") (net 2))
 (segment (start 108.3 90.5809) (end 118.0019 100.2828) (width 2) (layer "B.Cu") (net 2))
 (segment (start 117.475 105.9) (end 117.9499 105.9) (width 2) (layer "B.Cu") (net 2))
 (segment (start 145.65 112.1) (end 150.735 112.1) (width 2) (layer "B.Cu") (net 19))
 (segment (start 143.05 109.5) (end 145.65 112.1) (width 2) (layer "B.Cu") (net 19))
 (segment (start 143.05 102.35) (end 143.05 109.5) (width 2) (layer "B.Cu") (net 19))
 (segment (start 114.25 71.5) (end 114.25 94.48029) (width 0.5) (layer "B.Cu") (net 8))
 (segment (start 114.25 94.48029) (end 119.4519 99.68219) (width 0.5) (layer "B.Cu") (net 8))
 (segment (start 119.4519 99.68219) (end 119.4519 99.7019) (width 0.5) (layer "B.Cu") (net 8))
 (segment (start 120.01 100.26) (end 122.36 100.26) (width 0.5) (layer "B.Cu") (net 8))
 (segment (start 117.2 68.55) (end 114.25 71.5) (width 0.5) (layer "B.Cu") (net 8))
 (segment (start 124.15 68.55) (end 117.2 68.55) (width 0.5) (layer "B.Cu") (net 8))
 (segment (start 119.4519 99.7019) (end 120.01 100.26) (width 0.5) (layer "B.Cu") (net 8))
 (segment (start 122.869992 74.030008) (end 123.27 73.63) (width 0.5) (layer "B.Cu") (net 6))
 (segment (start 122.4 83.3025) (end 122.4 74.93067) (width 0.5) (layer "B.Cu") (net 6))
 (segment (start 122.869992 74.491331) (end 122.869992 74.030008) (width 0.5) (layer "B.Cu") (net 6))
 (segment (start 123.27 73.63) (end 124.15 73.63) (width 0.5) (layer "B.Cu") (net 6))
 (segment (start 122.36 105.34) (end 123.76 105.34) (width 0.5) (layer "B.Cu") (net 6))
 (segment (start 125.1064 86.0089) (end 122.4 83.3025) (width 0.5) (layer "B.Cu") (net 6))
 (segment (start 122.4 74.93067) (end 122.430653 74.93067) (width 0.5) (layer "B.Cu") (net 6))
 (segment (start 122.430653 74.93067) (end 122.869992 74.491331) (width 0.5) (layer "B.Cu") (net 6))
 (segment (start 125.1064 103.9936) (end 125.1064 86.0089) (width 0.5) (layer "B.Cu") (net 6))
 (segment (start 123.76 105.34) (end 125.1064 103.9936) (width 0.5) (layer "B.Cu") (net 6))
 (segment (start 123.6498 86.5322) (end 123.6498 97.5002) (width 0.5) (layer "B.Cu") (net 7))
 (segment (start 123.43 97.72) (end 122.36 97.72) (width 0.5) (layer "B.Cu") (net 7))
 (segment (start 122.61 71.09) (end 121 72.7) (width 0.5) (layer "B.Cu") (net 7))
 (segment (start 121 83.8824) (end 123.6498 86.5322) (width 0.5) (layer "B.Cu") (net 7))
 (segment (start 124.15 71.09) (end 122.61 71.09) (width 0.5) (layer "B.Cu") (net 7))
 (segment (start 121 72.7) (end 121 83.8824) (width 0.5) (layer "B.Cu") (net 7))
 (segment (start 123.6498 97.5002) (end 123.43 97.72) (width 0.5) (layer "B.Cu") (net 7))
 (segment (start 123.29668 76.17) (end 122.9054 75.77872) (width 0.5) (layer "F.Cu") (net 5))
 (segment (start 122.9054 74.966078) (end 122.119992 74.18067) (width 0.5) (layer "F.Cu") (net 5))
 (segment (start 124.15 76.17) (end 123.29668 76.17) (width 0.5) (layer "F.Cu") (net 5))
 (segment (start 122.9054 75.77872) (end 122.9054 74.966078) (width 0.5) (layer "F.Cu") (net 5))
 (via (at 122.119992 74.18067) (size 0.6) (drill 0.3) (layers "F.Cu" "B.Cu") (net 5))
 (segment (start 121.7 74.600662) (end 121.7 83.59245) (width 0.5) (layer "B.Cu") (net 5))
 (segment (start 122.119992 74.18067) (end 121.7 74.600662) (width 0.5) (layer "B.Cu") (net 5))
 (segment (start 124.4047 86.29715) (end 124.4047 101.9453) (width 0.5) (layer "B.Cu") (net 5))
 (segment (start 124.4047 101.9453) (end 123.55 102.8) (width 0.5) (layer "B.Cu") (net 5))
 (segment (start 123.55 102.8) (end 122.36 102.8) (width 0.5) (layer "B.Cu") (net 5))
 (segment (start 121.7 83.59245) (end 124.4047 86.29715) (width 0.5) (layer "B.Cu") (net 5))
 (segment (start 117.7 88.05) (end 119.75 90.1) (width 0.5) (layer "F.Cu") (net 20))
 (segment (start 119.75 90.1) (end 122.36 90.1) (width 0.5) (layer "F.Cu") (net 20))
 (segment (start 117.7 81.2) (end 117.7 88.05) (width 0.5) (layer "F.Cu") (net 20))
 (segment (start 120.3 86.9) (end 120.96 87.56) (width 0.5) (layer "B.Cu") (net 21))
 (segment (start 117.7 78.66) (end 119.31 78.66) (width 0.5) (layer "B.Cu") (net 21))
 (segment (start 119.31 78.66) (end 120.3 79.65) (width 0.5) (layer "B.Cu") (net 21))
 (segment (start 120.3 79.65) (end 120.3 86.9) (width 0.5) (layer "B.Cu") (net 21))
 (segment (start 120.96 87.56) (end 122.36 87.56) (width 0.5) (layer "B.Cu") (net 21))
 (segment (start 119.65 93.91) (end 130.01 93.91) (width 0.5) (layer "F.Cu") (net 10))
 (segment (start 103.05 78.66) (end 104.4 78.66) (width 0.5) (layer "F.Cu") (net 10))
 (segment (start 131.28 95.18) (end 137.6 95.18) (width 0.5) (layer "F.Cu") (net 10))
 (segment (start 130.01 93.91) (end 131.28 95.18) (width 0.5) (layer "F.Cu") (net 10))
 (segment (start 104.4 78.66) (end 119.65 93.91) (width 0.5) (layer "F.Cu") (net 10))
 (segment (start 103.05 76.12) (end 104.4 76.12) (width 0.5) (layer "F.Cu") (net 11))
 (segment (start 104.4 76.12) (end 119.65 91.37) (width 0.5) (layer "F.Cu") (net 11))
 (segment (start 130.32 91.37) (end 131.59 92.64) (width 0.5) (layer "F.Cu") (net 11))
 (segment (start 131.59 92.64) (end 137.6 92.64) (width 0.5) (layer "F.Cu") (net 11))
 (segment (start 119.65 91.37) (end 130.32 91.37) (width 0.5) (layer "F.Cu") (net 11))
 (segment (start 129.85 96.45) (end 131.12 97.72) (width 0.5) (layer "F.Cu") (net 9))
 (segment (start 104.4 81.2) (end 119.65 96.45) (width 0.5) (layer "F.Cu") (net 9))
 (segment (start 103.05 81.2) (end 104.4 81.2) (width 0.5) (layer "F.Cu") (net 9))
 (segment (start 119.65 96.45) (end 129.85 96.45) (width 0.5) (layer "F.Cu") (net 9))
 (segment (start 131.12 97.72) (end 137.6 97.72) (width 0.5) (layer "F.Cu") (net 9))
 (segment (start 133.9 89.3) (end 133.9 87.91005) (width 0.5) (layer "F.Cu") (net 4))
 (segment (start 139.859669 81.950381) (end 139.859669 79.190331) (width 0.5) (layer "F.Cu") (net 4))
 (segment (start 133.9 87.91005) (end 139.859669 81.950381) (width 0.5) (layer "F.Cu") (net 4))
 (via (at 133.9 89.3) (size 0.6) (drill 0.3) (layers "F.Cu" "B.Cu") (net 4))
 (via (at 139.859669 79.190331) (size 0.6) (drill 0.3) (layers "F.Cu" "B.Cu") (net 4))
 (segment (start 133.9 102.77137) (end 133.9 89.3) (width 0.5) (layer "B.Cu") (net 4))
 (segment (start 137.6 105.34) (end 136.46863 105.34) (width 0.5) (layer "B.Cu") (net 4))
 (segment (start 139.08 73.33) (end 137.6 73.33) (width 0.5) (layer "B.Cu") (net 4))
 (segment (start 139.85 74.1) (end 139.08 73.33) (width 0.5) (layer "B.Cu") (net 4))
 (segment (start 139.85 79.180662) (end 139.85 74.1) (width 0.5) (layer "B.Cu") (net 4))
 (segment (start 139.859669 79.190331) (end 139.85 79.180662) (width 0.5) (layer "B.Cu") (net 4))
 (segment (start 136.46863 105.34) (end 133.9 102.77137) (width 0.5) (layer "B.Cu") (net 4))
 (segment (start 134.7285 89.3) (end 134.7285 88.0715) (width 0.5) (layer "F.Cu") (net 3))
 (segment (start 141.2 78.26066) (end 139.85 76.91066) (width 0.5) (layer "F.Cu") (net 3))
 (segment (start 141.2 82.45) (end 141.2 78.26066) (width 0.5) (layer "F.Cu") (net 3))
 (segment (start 134.7285 88.0715) (end 137.15 85.65) (width 0.5) (layer "F.Cu") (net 3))
 (segment (start 137.15 85.65) (end 138 85.65) (width 0.5) (layer "F.Cu") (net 3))
 (segment (start 138 85.65) (end 141.2 82.45) (width 0.5) (layer "F.Cu") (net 3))
 (segment (start 139.85 76.35) (end 139.37 75.87) (width 0.5) (layer "F.Cu") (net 3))
 (segment (start 139.85 76.91066) (end 139.85 76.35) (width 0.5) (layer "F.Cu") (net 3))
 (segment (start 139.37 75.87) (end 137.6 75.87) (width 0.5) (layer "F.Cu") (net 3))
 (via (at 134.7285 89.3) (size 0.6) (drill 0.3) (layers "F.Cu" "B.Cu") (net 3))
 (segment (start 134.7285 89.3) (end 134.7285 101.8285) (width 0.5) (layer "B.Cu") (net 3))
 (segment (start 134.7285 101.8285) (end 135.7 102.8) (width 0.5) (layer "B.Cu") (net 3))
 (segment (start 135.7 102.8) (end 137.6 102.8) (width 0.5) (layer "B.Cu") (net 3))
 (segment (start 140.2191 112.1809) (end 140.2191 96.6409) (width 0.5) (layer "B.Cu") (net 18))
 (segment (start 137.6 112.96) (end 139.44 112.96) (width 0.5) (layer "B.Cu") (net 18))
 (segment (start 140.2191 96.6409) (end 143.1 93.76) (width 0.5) (layer "B.Cu") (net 18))
 (segment (start 139.44 112.96) (end 140.2191 112.1809) (width 0.5) (layer "B.Cu") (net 18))
 (segment (start 141.2 99.55) (end 143.1 97.65) (width 0.5) (layer "B.Cu") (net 17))
 (segment (start 141.2 114.1) (end 141.2 99.55) (width 0.5) (layer "B.Cu") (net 17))
 (segment (start 143.1 97.65) (end 143.1 96.3) (width 0.5) (layer "B.Cu") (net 17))
 (segment (start 137.6 115.5) (end 139.8 115.5) (width 0.5) (layer "B.Cu") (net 17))
 (segment (start 139.8 115.5) (end 141.2 114.1) (width 0.5) (layer "B.Cu") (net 17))
 (segment (start 116.03 110.43) (end 116.03 108.5) (width 0.5) (layer "F.Cu") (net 12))
 (segment (start 126.19 111.67) (end 117.27 111.67) (width 0.5) (layer "F.Cu") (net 12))
 (segment (start 117.27 111.67) (end 116.03 110.43) (width 0.5) (layer "F.Cu") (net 12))
 (segment (start 137.6 100.26) (end 126.19 111.67) (width 0.5) (layer "F.Cu") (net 12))
 (segment (start 119.4838 100.6662) (end 104.09385 100.6662) (width 0.5) (layer "F.Cu") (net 15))
 (segment (start 119.849997 97.2) (end 119.85 97.200003) (width 0.5) (layer "F.Cu") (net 15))
 (segment (start 104.09385 100.6662) (end 102.9466 101.81345) (width 0.5) (layer "F.Cu") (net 15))
 (segment (start 119.85 100.3) (end 119.4838 100.6662) (width 0.5) (layer "F.Cu") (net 15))
 (segment (start 119.85 97.200003) (end 119.85 100.3) (width 0.5) (layer "F.Cu") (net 15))
 (segment (start 107.7 111) (end 108.41 110.29) (width 0.5) (layer "F.Cu") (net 15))
 (segment (start 102.9466 110.0466) (end 103.9 111) (width 0.5) (layer "F.Cu") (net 15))
 (segment (start 102.9466 101.81345) (end 102.9466 110.0466) (width 0.5) (layer "F.Cu") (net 15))
 (segment (start 108.41 110.29) (end 108.41 108.5) (width 0.5) (layer "F.Cu") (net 15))
 (segment (start 103.9 111) (end 107.7 111) (width 0.5) (layer "F.Cu") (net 15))
 (via (at 119.849997 97.2) (size 0.6) (drill 0.3) (layers "F.Cu" "B.Cu") (free yes) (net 15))
 (segment (start 119.849997 97.2) (end 119.769669 97.119672) (width 0.5) (layer "B.Cu") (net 15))
 (segment (start 119.769669 97.119672) (end 119.769669 93.580331) (width 0.5) (layer "B.Cu") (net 15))
 (segment (start 120.71 92.64) (end 122.36 92.64) (width 0.5) (layer "B.Cu") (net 15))
 (segment (start 119.769669 93.580331) (end 120.71 92.64) (width 0.5) (layer "B.Cu") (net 15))
 (segment (start 139.05 104.05) (end 139.5 103.6) (width 0.5) (layer "F.Cu") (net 13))
 (segment (start 139.5 92) (end 137.6 90.1) (width 0.5) (layer "F.Cu") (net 13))
 (segment (start 115.81 114.21) (end 126.04 114.21) (width 0.5) (layer "F.Cu") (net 13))
 (segment (start 113.51 111.91) (end 115.81 114.21) (width 0.5) (layer "F.Cu") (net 13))
 (segment (start 126.04 114.21) (end 136.2 104.05) (width 0.5) (layer "F.Cu") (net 13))
 (segment (start 113.49 108.5) (end 113.51 108.52) (width 0.5) (layer "F.Cu") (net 13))
 (segment (start 136.2 104.05) (end 139.05 104.05) (width 0.5) (layer "F.Cu") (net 13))
 (segment (start 113.51 108.52) (end 113.51 111.91) (width 0.5) (layer "F.Cu") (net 13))
 (segment (start 139.5 103.6) (end 139.5 92) (width 0.5) (layer "F.Cu") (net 13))
 (segment (start 110.97 108.55) (end 110.95 108.57) (width 0.5) (layer "F.Cu") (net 14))
 (segment (start 115.9 116.75) (end 126.2 116.75) (width 0.5) (layer "F.Cu") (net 14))
 (segment (start 136.36 106.59) (end 139.36 106.59) (width 0.5) (layer "F.Cu") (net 14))
 (segment (start 140.2 105.75) (end 140.2 90.16) (width 0.5) (layer "F.Cu") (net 14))
 (segment (start 110.95 111.8) (end 115.9 116.75) (width 0.5) (layer "F.Cu") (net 14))
 (segment (start 139.36 106.59) (end 140.2 105.75) (width 0.5) (layer "F.Cu") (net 14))
 (segment (start 140.2 90.16) (end 137.6 87.56) (width 0.5) (layer "F.Cu") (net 14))
 (segment (start 126.2 116.75) (end 136.36 106.59) (width 0.5) (layer "F.Cu") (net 14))
 (segment (start 110.95 108.57) (end 110.95 111.8) (width 0.5) (layer "F.Cu") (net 14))
 (segment (start 120.65 100.7) (end 119.9838 101.3662) (width 0.5) (layer "F.Cu") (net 16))
 (segment (start 103.6466 102.1034) (end 103.6466 108.2466) (width 0.5) (layer "F.Cu") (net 16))
 (segment (start 104.3838 101.3662) (end 103.6466 102.1034) (width 0.5) (layer "F.Cu") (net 16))
 (segment (start 103.9 108.5) (end 105.87 108.5) (width 0.5) (layer "F.Cu") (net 16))
 (segment (start 119.9838 101.3662) (end 104.3838 101.3662) (width 0.5) (layer "F.Cu") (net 16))
 (segment (start 120.65 97.2) (end 120.65 100.7) (width 0.5) (layer "F.Cu") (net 16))
 (segment (start 103.6466 108.2466) (end 103.9 108.5) (width 0.5) (layer "F.Cu") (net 16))
 (via (at 120.65 97.2) (size 0.6) (drill 0.3) (layers "F.Cu" "B.Cu") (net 16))
 (segment (start 120.65 95.8) (end 121.27 95.18) (width 0.5) (layer "B.Cu") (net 16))
 (segment (start 121.27 95.18) (end 122.36 95.18) (width 0.5) (layer "B.Cu") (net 16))
 (segment (start 120.65 97.2) (end 120.65 95.8) (width 0.5) (layer "B.Cu") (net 16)))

